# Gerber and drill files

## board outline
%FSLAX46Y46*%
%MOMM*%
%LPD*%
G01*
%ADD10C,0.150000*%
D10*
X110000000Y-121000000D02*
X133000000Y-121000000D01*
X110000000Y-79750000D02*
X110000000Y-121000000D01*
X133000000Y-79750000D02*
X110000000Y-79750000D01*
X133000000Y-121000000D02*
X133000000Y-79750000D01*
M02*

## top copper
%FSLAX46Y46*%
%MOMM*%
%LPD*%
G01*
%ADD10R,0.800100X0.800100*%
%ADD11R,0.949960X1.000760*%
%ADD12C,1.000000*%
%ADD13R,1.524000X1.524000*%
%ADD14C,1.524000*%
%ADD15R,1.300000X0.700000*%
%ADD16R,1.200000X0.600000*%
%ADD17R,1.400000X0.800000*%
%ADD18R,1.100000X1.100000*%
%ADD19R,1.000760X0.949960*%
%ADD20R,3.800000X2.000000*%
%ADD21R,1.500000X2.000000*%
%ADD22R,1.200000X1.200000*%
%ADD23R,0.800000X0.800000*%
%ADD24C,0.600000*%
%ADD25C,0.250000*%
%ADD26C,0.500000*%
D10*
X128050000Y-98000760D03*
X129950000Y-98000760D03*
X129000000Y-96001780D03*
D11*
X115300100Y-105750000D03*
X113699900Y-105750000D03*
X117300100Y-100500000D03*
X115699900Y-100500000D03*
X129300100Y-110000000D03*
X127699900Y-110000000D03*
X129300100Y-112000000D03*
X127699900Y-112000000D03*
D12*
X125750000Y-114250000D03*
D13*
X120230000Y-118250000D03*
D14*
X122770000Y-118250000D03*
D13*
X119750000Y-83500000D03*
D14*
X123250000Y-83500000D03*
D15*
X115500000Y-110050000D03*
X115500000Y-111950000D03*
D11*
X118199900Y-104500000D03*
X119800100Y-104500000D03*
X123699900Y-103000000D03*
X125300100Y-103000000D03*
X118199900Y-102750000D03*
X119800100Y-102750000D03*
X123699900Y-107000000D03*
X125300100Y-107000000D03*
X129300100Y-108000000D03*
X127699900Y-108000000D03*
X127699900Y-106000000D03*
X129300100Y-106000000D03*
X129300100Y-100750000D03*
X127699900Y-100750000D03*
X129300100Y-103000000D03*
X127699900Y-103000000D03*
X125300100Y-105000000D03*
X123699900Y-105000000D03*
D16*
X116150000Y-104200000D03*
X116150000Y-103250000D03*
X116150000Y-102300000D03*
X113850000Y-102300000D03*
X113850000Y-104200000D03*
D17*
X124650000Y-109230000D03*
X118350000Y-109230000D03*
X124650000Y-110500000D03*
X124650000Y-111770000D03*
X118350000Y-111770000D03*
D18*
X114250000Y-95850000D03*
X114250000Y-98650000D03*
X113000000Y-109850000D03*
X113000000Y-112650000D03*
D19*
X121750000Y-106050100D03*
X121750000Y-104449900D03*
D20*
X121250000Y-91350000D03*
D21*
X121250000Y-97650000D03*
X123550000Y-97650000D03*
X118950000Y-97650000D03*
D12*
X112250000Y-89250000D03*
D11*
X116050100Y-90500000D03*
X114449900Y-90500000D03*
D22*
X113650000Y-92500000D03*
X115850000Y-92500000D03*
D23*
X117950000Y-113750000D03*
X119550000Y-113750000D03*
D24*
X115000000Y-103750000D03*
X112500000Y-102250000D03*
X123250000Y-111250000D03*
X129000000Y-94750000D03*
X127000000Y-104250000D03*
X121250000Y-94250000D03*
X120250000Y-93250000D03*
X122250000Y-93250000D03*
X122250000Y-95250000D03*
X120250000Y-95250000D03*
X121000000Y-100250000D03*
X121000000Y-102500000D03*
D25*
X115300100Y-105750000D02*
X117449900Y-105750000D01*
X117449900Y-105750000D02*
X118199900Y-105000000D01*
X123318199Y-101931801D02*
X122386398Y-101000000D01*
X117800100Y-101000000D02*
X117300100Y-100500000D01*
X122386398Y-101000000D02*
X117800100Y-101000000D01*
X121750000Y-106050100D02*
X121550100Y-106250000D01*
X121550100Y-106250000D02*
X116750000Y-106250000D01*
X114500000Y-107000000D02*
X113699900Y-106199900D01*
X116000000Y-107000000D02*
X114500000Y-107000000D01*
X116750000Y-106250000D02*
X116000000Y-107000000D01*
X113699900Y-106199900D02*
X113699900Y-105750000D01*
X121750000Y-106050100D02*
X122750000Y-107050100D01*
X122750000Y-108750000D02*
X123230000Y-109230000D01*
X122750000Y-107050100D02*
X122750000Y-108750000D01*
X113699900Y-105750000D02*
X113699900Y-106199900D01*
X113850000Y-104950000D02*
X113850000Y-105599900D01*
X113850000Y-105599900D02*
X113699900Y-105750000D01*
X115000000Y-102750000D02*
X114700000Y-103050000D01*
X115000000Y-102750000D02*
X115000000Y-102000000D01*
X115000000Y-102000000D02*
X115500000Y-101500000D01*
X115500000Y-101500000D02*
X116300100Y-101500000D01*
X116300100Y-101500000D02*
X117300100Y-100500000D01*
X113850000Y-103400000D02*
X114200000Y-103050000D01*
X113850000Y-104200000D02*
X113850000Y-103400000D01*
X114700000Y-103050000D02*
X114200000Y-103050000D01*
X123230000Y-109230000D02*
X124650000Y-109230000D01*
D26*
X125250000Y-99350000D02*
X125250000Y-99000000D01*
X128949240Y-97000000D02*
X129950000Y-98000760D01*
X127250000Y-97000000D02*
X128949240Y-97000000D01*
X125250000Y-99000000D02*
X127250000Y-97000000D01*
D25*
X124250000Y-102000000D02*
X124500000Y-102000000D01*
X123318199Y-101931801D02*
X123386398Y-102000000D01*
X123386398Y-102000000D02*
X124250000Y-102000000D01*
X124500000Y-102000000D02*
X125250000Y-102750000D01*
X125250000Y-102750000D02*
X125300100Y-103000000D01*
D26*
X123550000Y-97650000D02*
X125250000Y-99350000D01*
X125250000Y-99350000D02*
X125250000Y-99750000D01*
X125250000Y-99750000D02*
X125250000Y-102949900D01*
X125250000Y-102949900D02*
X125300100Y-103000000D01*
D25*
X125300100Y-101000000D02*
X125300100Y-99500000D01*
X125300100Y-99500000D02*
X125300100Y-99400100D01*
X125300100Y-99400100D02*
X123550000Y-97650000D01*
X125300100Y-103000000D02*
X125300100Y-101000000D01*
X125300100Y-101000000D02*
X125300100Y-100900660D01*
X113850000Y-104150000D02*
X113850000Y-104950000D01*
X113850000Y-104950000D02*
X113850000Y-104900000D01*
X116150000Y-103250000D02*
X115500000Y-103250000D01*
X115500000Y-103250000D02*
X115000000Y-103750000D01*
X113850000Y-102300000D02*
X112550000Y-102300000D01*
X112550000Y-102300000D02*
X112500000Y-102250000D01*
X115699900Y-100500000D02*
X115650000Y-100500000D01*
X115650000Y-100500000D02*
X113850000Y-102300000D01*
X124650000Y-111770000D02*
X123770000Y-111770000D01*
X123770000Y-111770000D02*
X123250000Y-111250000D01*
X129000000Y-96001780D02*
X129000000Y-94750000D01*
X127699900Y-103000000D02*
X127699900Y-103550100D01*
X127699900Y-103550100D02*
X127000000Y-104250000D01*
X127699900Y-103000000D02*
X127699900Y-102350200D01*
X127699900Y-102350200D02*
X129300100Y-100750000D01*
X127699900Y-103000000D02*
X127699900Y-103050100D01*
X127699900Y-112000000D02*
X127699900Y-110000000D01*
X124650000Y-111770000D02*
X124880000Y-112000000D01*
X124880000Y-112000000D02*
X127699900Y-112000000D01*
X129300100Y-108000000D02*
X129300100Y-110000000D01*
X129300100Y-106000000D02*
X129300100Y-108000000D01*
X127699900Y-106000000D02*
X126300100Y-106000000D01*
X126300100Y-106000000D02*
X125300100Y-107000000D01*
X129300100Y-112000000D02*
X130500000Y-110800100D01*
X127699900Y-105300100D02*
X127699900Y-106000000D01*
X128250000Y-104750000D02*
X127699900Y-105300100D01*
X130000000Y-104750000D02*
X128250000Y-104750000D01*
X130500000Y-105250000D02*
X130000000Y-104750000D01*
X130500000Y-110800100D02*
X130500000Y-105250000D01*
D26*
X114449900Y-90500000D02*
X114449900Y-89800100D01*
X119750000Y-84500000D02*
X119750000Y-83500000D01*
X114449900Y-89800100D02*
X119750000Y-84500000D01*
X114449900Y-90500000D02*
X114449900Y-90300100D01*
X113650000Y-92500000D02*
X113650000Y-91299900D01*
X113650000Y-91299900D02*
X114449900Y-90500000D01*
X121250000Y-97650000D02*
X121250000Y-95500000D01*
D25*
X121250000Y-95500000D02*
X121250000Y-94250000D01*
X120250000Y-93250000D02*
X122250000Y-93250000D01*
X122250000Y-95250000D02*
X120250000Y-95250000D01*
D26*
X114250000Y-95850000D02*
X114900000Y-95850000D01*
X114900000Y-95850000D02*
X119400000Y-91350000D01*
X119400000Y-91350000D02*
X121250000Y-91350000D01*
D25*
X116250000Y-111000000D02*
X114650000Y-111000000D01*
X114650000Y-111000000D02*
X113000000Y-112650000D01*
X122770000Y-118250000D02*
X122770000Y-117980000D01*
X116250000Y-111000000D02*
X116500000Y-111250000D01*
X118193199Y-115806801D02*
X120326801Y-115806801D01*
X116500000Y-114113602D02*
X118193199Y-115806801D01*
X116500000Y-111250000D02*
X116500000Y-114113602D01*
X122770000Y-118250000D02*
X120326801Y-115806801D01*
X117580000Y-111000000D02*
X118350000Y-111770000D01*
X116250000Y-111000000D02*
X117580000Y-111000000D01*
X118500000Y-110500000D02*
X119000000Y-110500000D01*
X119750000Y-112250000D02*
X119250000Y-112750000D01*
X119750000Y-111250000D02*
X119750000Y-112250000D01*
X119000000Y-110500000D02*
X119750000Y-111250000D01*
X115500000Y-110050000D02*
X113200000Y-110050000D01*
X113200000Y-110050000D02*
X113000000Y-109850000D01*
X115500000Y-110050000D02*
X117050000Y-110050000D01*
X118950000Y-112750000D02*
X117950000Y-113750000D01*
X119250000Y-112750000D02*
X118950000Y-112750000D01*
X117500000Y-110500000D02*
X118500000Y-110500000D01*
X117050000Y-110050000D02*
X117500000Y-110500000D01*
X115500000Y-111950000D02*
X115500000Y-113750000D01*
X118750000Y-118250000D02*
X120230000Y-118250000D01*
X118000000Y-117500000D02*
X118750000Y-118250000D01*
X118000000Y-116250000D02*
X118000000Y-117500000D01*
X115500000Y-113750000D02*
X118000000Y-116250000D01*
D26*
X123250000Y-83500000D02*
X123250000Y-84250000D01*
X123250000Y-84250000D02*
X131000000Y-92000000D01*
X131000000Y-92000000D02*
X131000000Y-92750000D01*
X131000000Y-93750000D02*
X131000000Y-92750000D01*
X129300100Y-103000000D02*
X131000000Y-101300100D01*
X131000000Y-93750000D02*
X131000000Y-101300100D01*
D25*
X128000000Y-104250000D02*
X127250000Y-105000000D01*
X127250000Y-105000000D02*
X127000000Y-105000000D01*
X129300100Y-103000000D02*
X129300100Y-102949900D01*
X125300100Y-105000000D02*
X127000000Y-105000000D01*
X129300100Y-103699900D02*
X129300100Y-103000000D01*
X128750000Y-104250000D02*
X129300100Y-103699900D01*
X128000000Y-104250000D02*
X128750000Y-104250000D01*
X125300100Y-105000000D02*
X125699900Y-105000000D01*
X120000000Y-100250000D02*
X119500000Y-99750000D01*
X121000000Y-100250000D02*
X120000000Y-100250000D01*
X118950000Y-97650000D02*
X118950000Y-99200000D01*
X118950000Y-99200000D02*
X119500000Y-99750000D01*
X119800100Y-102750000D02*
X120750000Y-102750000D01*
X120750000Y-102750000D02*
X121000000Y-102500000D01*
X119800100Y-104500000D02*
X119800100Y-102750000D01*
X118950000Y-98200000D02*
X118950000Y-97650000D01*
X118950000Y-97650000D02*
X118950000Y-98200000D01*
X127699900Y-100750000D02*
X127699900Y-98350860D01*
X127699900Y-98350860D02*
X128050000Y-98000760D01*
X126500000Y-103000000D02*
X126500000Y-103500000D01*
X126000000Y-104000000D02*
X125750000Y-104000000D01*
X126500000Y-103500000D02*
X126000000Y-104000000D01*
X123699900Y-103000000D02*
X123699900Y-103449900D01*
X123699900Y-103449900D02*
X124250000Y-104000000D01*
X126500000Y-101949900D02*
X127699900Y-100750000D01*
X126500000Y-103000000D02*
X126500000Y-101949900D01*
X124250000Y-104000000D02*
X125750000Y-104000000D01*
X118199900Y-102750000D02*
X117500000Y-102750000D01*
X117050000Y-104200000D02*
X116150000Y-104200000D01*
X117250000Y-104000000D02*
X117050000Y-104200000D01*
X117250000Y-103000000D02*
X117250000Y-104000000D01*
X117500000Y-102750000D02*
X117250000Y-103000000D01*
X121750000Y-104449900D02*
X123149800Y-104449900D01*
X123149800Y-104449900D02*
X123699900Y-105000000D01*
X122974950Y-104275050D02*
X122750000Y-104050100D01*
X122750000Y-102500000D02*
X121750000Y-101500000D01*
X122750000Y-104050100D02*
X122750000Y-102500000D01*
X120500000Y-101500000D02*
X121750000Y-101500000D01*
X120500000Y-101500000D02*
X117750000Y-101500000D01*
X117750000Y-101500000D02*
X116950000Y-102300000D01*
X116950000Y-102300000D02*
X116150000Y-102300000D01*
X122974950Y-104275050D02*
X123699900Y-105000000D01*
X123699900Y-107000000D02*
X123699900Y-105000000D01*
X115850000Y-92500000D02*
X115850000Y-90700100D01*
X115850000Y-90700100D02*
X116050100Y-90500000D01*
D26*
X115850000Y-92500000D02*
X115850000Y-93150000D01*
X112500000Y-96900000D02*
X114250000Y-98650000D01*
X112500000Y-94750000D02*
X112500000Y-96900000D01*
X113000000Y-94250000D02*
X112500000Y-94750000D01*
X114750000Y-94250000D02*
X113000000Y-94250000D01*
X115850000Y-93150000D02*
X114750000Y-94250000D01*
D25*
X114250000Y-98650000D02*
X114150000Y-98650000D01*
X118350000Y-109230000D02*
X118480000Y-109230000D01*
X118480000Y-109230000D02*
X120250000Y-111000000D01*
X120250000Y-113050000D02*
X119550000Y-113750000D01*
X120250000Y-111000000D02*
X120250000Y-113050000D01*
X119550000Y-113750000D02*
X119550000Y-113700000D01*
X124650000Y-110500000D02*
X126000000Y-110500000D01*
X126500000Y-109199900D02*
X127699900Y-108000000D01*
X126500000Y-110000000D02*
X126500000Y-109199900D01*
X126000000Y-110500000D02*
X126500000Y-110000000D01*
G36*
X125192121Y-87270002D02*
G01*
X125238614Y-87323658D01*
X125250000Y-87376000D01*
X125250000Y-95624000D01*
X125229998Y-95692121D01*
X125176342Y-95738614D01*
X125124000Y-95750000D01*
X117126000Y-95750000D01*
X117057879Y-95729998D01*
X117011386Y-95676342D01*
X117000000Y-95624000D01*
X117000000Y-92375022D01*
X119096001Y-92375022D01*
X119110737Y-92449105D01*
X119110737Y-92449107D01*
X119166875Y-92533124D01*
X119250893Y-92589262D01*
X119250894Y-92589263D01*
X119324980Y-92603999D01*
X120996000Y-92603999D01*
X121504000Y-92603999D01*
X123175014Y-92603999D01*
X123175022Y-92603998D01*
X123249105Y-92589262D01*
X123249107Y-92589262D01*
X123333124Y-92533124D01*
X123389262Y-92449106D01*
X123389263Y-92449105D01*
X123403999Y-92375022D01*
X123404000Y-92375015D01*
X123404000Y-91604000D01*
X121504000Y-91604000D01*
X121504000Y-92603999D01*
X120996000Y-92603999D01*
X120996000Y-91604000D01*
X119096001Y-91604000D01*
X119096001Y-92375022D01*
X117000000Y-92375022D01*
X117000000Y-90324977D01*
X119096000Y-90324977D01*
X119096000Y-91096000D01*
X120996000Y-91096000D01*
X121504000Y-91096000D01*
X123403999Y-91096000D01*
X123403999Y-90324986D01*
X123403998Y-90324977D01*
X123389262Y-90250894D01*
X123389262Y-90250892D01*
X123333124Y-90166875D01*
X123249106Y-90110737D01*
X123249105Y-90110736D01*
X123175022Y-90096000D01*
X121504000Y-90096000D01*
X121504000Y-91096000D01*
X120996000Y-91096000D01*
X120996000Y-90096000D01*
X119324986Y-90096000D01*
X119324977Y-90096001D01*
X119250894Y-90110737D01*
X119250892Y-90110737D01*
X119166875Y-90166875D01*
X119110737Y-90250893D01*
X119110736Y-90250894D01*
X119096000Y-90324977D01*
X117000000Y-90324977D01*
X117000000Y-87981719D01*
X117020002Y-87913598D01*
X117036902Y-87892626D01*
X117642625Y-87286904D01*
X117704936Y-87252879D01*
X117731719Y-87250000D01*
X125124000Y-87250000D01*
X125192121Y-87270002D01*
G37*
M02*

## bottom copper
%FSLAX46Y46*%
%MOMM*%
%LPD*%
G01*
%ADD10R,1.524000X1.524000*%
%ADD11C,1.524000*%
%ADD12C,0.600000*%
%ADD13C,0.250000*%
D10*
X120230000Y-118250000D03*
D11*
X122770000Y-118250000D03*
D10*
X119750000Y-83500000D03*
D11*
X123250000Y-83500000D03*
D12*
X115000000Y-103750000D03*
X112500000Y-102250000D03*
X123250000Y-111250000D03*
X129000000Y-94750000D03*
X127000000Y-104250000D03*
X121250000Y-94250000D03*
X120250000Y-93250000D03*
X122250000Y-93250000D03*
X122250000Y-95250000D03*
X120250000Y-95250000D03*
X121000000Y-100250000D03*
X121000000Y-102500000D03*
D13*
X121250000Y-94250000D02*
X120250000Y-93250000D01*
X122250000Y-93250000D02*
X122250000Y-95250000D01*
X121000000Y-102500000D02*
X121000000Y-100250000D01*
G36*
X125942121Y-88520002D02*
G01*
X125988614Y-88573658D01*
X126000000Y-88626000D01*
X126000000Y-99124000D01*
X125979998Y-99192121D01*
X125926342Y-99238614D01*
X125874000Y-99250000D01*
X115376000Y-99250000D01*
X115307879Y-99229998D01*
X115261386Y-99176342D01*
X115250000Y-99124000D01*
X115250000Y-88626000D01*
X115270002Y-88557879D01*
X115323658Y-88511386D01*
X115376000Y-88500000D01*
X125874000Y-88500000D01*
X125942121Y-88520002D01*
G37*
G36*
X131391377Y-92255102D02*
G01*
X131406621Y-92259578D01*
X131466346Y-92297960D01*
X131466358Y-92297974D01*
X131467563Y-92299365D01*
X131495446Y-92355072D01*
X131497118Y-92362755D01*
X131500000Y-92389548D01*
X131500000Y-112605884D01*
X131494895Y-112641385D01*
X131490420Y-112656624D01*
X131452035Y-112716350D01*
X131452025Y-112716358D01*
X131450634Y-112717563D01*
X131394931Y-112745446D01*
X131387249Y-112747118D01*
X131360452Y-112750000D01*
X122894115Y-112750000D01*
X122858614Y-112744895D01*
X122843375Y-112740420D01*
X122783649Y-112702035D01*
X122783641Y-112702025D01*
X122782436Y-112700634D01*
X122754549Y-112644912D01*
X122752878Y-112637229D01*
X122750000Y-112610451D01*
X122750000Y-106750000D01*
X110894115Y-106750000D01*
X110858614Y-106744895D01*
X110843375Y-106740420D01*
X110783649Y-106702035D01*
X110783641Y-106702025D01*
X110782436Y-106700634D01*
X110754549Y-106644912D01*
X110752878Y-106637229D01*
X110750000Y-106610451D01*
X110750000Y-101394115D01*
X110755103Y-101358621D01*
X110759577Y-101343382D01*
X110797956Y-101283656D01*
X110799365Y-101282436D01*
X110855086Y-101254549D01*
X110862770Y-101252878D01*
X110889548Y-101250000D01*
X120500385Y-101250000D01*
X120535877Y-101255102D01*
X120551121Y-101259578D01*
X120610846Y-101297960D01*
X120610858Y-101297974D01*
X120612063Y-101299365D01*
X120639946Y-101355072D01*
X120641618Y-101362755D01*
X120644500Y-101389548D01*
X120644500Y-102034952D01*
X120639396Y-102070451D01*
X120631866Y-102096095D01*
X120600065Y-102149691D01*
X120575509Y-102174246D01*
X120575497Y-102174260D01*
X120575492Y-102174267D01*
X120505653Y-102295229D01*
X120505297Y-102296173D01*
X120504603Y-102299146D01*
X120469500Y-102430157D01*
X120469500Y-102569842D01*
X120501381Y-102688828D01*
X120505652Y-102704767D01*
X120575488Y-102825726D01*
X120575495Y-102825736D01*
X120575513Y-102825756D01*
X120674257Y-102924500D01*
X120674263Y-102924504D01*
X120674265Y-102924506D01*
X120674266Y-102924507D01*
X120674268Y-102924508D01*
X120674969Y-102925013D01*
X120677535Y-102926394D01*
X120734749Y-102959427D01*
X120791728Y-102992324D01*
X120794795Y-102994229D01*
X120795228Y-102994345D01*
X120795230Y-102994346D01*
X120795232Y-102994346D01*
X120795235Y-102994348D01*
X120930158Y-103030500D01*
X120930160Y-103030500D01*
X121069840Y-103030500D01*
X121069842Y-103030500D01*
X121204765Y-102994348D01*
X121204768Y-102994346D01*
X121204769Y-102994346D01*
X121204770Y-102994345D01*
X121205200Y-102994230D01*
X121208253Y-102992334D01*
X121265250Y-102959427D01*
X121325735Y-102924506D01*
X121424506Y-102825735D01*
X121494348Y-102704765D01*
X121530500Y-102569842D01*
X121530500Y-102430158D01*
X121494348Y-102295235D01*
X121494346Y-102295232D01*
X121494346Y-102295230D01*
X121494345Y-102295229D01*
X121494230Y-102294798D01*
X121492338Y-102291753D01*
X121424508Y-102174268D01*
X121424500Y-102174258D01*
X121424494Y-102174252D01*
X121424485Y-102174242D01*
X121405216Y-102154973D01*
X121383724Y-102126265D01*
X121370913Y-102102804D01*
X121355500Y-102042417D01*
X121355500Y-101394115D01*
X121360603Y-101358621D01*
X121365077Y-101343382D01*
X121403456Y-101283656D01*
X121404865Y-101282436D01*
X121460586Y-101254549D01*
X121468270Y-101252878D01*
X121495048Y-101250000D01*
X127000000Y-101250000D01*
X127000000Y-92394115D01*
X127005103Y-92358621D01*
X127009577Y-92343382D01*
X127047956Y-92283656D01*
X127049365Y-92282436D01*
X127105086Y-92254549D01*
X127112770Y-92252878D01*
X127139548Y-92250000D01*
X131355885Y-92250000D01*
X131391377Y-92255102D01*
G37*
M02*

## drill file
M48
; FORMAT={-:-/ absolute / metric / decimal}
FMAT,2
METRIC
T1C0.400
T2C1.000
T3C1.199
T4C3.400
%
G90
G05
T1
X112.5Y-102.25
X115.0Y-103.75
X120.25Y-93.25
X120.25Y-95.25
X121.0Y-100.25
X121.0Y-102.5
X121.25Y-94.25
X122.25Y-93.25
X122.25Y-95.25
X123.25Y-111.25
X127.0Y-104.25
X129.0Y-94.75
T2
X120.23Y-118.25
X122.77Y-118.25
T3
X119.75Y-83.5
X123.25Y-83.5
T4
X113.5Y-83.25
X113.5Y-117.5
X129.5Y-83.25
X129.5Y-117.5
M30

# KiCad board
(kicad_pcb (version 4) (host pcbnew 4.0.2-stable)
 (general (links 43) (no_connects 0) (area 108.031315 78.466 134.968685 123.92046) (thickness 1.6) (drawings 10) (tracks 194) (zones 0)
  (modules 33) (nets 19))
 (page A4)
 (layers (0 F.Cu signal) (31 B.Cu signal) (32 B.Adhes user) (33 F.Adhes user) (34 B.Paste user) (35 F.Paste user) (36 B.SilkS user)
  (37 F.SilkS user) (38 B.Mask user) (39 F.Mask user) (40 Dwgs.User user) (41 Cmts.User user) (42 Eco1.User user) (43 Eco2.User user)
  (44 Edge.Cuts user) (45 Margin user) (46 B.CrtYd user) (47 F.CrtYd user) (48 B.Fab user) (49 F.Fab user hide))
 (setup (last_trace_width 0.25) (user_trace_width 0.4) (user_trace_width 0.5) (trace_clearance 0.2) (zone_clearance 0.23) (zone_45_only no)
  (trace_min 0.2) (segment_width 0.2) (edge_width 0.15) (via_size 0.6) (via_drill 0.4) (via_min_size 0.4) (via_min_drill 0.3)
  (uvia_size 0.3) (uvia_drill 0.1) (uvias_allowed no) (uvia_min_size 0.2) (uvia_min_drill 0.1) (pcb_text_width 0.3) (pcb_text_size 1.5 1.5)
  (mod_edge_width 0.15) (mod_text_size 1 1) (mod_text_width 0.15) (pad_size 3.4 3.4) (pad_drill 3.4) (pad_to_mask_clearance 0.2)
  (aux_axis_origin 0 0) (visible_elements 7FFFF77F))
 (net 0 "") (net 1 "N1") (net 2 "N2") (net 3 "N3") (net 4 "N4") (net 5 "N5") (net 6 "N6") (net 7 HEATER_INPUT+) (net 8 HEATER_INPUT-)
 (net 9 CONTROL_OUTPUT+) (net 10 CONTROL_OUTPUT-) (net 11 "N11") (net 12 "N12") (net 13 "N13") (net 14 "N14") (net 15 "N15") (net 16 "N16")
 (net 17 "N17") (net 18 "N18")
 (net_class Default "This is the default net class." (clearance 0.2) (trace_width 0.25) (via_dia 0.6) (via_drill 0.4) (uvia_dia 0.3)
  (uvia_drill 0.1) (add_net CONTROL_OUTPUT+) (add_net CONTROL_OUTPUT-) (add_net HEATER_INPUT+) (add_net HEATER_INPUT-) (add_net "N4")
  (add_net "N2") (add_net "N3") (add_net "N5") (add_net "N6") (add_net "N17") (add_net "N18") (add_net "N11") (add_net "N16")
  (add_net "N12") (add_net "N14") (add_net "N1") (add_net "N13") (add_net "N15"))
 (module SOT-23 (layer F.Cu) (at 129 97)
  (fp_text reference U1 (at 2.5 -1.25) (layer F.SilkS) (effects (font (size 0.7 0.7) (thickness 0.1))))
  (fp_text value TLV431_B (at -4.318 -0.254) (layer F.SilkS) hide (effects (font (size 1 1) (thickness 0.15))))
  (pad 1 smd rect (at -0.95 1.00076) (size 0.8001 0.8001) (layers F.Cu F.Paste F.Mask) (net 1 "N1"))
  (pad 2 smd rect (at 0.95 1.00076) (size 0.8001 0.8001) (layers F.Cu F.Paste F.Mask) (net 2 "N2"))
  (pad 3 smd rect (at 0 -0.99822) (size 0.8001 0.8001) (layers F.Cu F.Paste F.Mask) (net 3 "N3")))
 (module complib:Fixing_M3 (layer F.Cu) (at 129.5 117.5)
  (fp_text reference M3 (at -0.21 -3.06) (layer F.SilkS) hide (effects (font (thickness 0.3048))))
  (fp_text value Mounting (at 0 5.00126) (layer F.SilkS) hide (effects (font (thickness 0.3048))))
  (pad "" np_thru_hole circle (at 0 0) (size 3.4 3.4) (drill 3.4) (layers *.Cu *.Mask F.SilkS)))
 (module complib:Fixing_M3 (layer F.Cu) (at 113.5 83.25)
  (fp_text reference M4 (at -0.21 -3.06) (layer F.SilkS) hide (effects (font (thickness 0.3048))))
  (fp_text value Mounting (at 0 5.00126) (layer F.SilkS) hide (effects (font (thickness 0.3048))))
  (pad "" np_thru_hole circle (at 0 0) (size 3.4 3.4) (drill 3.4) (layers *.Cu *.Mask F.SilkS)))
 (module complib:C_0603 (layer F.Cu) (at 114.5 105.75)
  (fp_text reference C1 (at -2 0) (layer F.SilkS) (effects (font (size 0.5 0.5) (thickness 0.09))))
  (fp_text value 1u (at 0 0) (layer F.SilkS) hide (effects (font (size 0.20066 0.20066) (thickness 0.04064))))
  (pad 1 smd rect (at 0.8001 0) (size 0.94996 1.00076) (layers F.Cu F.Paste F.Mask) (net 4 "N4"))
  (pad 2 smd rect (at -0.8001 0) (size 0.94996 1.00076) (layers F.Cu F.Paste F.Mask) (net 2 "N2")))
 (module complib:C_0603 (layer F.Cu) (at 116.5 100.5)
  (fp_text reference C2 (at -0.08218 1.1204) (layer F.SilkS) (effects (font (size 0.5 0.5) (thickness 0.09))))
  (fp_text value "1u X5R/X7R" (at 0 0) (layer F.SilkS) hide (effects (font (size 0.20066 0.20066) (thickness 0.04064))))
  (pad 1 smd rect (at 0.8001 0) (size 0.94996 1.00076) (layers F.Cu F.Paste F.Mask) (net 2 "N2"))
  (pad 2 smd rect (at -0.8001 0) (size 0.94996 1.00076) (layers F.Cu F.Paste F.Mask) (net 3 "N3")))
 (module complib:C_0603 (layer F.Cu) (at 128.5 110)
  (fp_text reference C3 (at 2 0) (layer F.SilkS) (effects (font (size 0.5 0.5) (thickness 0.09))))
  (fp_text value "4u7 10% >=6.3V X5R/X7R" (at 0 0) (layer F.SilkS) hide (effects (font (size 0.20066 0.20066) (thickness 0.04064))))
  (pad 1 smd rect (at 0.8001 0) (size 0.94996 1.00076) (layers F.Cu F.Paste F.Mask) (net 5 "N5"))
  (pad 2 smd rect (at -0.8001 0) (size 0.94996 1.00076) (layers F.Cu F.Paste F.Mask) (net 3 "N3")))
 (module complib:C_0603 (layer F.Cu) (at 128.5 112)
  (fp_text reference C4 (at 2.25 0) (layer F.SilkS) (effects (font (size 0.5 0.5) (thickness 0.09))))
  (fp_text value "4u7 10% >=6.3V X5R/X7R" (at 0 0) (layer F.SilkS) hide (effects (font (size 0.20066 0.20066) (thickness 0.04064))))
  (pad 1 smd rect (at 0.8001 0) (size 0.94996 1.00076) (layers F.Cu F.Paste F.Mask) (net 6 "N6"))
  (pad 2 smd rect (at -0.8001 0) (size 0.94996 1.00076) (layers F.Cu F.Paste F.Mask) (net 3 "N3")))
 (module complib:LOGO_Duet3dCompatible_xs (layer B.Cu) (at 117.25 101.75 270)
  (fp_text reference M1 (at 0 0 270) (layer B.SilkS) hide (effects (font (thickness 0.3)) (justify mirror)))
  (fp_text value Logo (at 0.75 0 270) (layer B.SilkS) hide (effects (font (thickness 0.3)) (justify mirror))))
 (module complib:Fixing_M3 (layer F.Cu) (at 129.5 83.25)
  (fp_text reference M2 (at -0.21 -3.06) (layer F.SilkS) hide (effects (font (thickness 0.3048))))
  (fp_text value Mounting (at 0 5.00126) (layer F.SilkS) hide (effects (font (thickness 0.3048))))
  (pad "" np_thru_hole circle (at 0 0) (size 3.4 3.4) (drill 3.4) (layers *.Cu *.Mask F.SilkS)))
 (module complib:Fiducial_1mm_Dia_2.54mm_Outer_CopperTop (layer F.Cu) (at 125.75 114.25)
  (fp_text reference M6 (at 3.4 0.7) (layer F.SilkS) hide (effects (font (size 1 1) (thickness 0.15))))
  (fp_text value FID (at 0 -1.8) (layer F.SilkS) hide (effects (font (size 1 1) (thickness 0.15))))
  (pad ~ smd circle (at 0 0) (size 1 1) (layers F.Cu F.Mask) (solder_mask_margin 0.77) (clearance 0.77)))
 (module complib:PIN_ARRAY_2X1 (layer F.Cu) (at 121.5 118.25)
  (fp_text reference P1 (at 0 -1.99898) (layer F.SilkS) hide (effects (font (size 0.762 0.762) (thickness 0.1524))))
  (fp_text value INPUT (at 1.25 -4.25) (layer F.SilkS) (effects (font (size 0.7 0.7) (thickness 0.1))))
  (pad 1 thru_hole rect (at -1.27 0) (size 1.524 1.524) (drill 1) (layers *.Cu *.Mask F.SilkS) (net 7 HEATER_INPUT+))
  (pad 2 thru_hole circle (at 1.27 0) (size 1.524 1.524) (drill 1) (layers *.Cu *.Mask F.SilkS) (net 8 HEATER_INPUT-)))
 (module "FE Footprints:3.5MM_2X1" (layer F.Cu) (at 121.5 83.5)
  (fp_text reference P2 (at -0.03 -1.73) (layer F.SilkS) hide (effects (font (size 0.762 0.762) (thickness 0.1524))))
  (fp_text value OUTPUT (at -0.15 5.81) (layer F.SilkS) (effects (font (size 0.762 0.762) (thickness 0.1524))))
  (pad 1 thru_hole rect (at -1.75 0) (size 1.524 1.524) (drill 1.19888) (layers *.Cu *.Mask F.SilkS) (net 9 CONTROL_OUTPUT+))
  (pad 2 thru_hole circle (at 1.75 0) (size 1.524 1.524) (drill 1.19888) (layers *.Cu *.Mask F.SilkS) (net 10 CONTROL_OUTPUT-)))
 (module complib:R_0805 (layer F.Cu) (at 115.5 111 270)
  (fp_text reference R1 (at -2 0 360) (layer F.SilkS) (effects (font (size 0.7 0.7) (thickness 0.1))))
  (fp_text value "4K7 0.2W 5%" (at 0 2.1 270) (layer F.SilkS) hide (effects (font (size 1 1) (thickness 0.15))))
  (pad 1 smd rect (at -0.95 0 270) (size 0.7 1.3) (layers F.Cu F.Paste F.Mask) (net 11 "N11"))
  (pad 2 smd rect (at 0.95 0 270) (size 0.7 1.3) (layers F.Cu F.Paste F.Mask) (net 7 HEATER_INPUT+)))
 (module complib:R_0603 (layer F.Cu) (at 119 104.5)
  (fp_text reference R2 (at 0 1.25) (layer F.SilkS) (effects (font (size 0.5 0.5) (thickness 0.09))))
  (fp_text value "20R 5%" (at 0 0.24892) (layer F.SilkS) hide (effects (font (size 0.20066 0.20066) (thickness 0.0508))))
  (pad 1 smd rect (at -0.8001 0) (size 0.94996 1.00076) (layers F.Cu F.Paste F.Mask) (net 4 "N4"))
  (pad 2 smd rect (at 0.8001 0) (size 0.94996 1.00076) (layers F.Cu F.Paste F.Mask) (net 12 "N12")))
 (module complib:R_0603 (layer F.Cu) (at 124.5 103)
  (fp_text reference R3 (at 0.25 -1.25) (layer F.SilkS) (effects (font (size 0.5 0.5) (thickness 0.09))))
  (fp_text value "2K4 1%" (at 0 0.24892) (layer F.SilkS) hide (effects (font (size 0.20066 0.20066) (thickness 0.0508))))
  (pad 1 smd rect (at -0.8001 0) (size 0.94996 1.00076) (layers F.Cu F.Paste F.Mask) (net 1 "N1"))
  (pad 2 smd rect (at 0.8001 0) (size 0.94996 1.00076) (layers F.Cu F.Paste F.Mask) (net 2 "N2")))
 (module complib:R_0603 (layer F.Cu) (at 119 102.75)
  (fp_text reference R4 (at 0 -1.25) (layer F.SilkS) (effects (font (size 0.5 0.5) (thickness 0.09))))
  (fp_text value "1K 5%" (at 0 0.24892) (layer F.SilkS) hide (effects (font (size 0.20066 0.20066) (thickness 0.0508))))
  (pad 1 smd rect (at -0.8001 0) (size 0.94996 1.00076) (layers F.Cu F.Paste F.Mask) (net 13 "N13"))
  (pad 2 smd rect (at 0.8001 0) (size 0.94996 1.00076) (layers F.Cu F.Paste F.Mask) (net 12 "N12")))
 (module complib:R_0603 (layer F.Cu) (at 124.5 107)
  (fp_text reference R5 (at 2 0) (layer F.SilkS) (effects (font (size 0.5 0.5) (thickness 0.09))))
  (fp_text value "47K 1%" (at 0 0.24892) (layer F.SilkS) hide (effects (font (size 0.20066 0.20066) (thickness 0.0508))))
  (pad 1 smd rect (at -0.8001 0) (size 0.94996 1.00076) (layers F.Cu F.Paste F.Mask) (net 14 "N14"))
  (pad 2 smd rect (at 0.8001 0) (size 0.94996 1.00076) (layers F.Cu F.Paste F.Mask) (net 6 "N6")))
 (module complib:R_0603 (layer F.Cu) (at 128.5 108 180)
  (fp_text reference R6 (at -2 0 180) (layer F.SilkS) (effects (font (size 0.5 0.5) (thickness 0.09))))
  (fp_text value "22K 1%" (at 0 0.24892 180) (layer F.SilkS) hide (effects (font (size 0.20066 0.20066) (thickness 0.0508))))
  (pad 1 smd rect (at -0.8001 0 180) (size 0.94996 1.00076) (layers F.Cu F.Paste F.Mask) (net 5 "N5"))
  (pad 2 smd rect (at 0.8001 0 180) (size 0.94996 1.00076) (layers F.Cu F.Paste F.Mask) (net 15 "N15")))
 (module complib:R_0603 (layer F.Cu) (at 128.5 106)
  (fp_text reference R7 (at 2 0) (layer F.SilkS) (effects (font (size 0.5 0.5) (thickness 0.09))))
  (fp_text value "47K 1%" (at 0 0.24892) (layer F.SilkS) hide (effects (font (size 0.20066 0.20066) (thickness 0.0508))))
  (pad 1 smd rect (at -0.8001 0) (size 0.94996 1.00076) (layers F.Cu F.Paste F.Mask) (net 6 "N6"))
  (pad 2 smd rect (at 0.8001 0) (size 0.94996 1.00076) (layers F.Cu F.Paste F.Mask) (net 5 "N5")))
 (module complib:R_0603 (layer F.Cu) (at 128.5 100.75 180)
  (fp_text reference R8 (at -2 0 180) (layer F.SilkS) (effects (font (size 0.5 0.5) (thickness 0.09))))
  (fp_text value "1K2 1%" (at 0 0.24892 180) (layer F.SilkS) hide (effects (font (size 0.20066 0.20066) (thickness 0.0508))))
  (pad 1 smd rect (at -0.8001 0 180) (size 0.94996 1.00076) (layers F.Cu F.Paste F.Mask) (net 3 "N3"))
  (pad 2 smd rect (at 0.8001 0 180) (size 0.94996 1.00076) (layers F.Cu F.Paste F.Mask) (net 1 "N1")))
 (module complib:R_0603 (layer F.Cu) (at 128.5 103 180)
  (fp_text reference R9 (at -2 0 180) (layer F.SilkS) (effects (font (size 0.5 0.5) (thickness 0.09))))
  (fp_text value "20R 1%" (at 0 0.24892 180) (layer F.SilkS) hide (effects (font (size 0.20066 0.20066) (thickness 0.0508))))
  (pad 1 smd rect (at -0.8001 0 180) (size 0.94996 1.00076) (layers F.Cu F.Paste F.Mask) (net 10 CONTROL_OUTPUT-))
  (pad 2 smd rect (at 0.8001 0 180) (size 0.94996 1.00076) (layers F.Cu F.Paste F.Mask) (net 3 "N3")))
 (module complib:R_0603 (layer F.Cu) (at 124.5 105 180)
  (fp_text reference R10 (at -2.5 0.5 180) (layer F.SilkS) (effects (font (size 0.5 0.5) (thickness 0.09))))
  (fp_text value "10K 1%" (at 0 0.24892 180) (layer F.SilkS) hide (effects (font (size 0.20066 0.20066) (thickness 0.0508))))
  (pad 1 smd rect (at -0.8001 0 180) (size 0.94996 1.00076) (layers F.Cu F.Paste F.Mask) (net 10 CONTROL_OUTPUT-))
  (pad 2 smd rect (at 0.8001 0 180) (size 0.94996 1.00076) (layers F.Cu F.Paste F.Mask) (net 14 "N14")))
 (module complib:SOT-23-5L (layer F.Cu) (at 115 103.25 180)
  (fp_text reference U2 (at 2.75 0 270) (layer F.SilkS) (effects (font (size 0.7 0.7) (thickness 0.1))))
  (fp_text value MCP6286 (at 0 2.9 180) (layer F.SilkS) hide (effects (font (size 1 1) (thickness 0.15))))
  (pad 1 smd rect (at -1.15 -0.95 180) (size 1.2 0.6) (layers F.Cu F.Paste F.Mask) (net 13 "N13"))
  (pad 2 smd rect (at -1.15 0 180) (size 1.2 0.6) (layers F.Cu F.Paste F.Mask) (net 3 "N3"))
  (pad 3 smd rect (at -1.15 0.95 180) (size 1.2 0.6) (layers F.Cu F.Paste F.Mask) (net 14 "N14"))
  (pad 4 smd rect (at 1.15 0.95 180) (size 1.2 0.6) (layers F.Cu F.Paste F.Mask) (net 3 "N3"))
  (pad 5 smd rect (at 1.15 -0.95 180) (size 1.2 0.6) (layers F.Cu F.Paste F.Mask) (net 2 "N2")))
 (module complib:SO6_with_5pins (layer F.Cu) (at 121.5 110.5 270)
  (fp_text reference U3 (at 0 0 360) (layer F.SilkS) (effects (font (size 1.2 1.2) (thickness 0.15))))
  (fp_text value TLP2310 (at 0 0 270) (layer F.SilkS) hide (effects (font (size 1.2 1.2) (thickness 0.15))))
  (pad 6 smd rect (at -1.27 -3.15 270) (size 0.8 1.4) (layers F.Cu F.Paste F.Mask) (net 2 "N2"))
  (pad 1 smd rect (at -1.27 3.15 270) (size 0.8 1.4) (layers F.Cu F.Paste F.Mask) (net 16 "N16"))
  (pad 5 smd rect (at 0 -3.15 270) (size 0.8 1.4) (layers F.Cu F.Paste F.Mask) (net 15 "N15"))
  (pad 4 smd rect (at 1.27 -3.15 270) (size 0.8 1.4) (layers F.Cu F.Paste F.Mask) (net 3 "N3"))
  (pad 3 smd rect (at 1.27 3.15 270) (size 0.8 1.4) (layers F.Cu F.Paste F.Mask) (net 8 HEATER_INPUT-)))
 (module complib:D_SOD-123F (layer F.Cu) (at 114.25 97.25 270)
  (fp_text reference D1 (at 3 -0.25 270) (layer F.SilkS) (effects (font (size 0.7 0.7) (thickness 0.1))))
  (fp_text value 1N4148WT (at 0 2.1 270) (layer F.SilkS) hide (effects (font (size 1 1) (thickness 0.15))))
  (pad 1 smd rect (at -1.4 0 270) (size 1.1 1.1) (layers F.Cu F.Paste F.Mask) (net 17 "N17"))
  (pad 2 smd rect (at 1.4 0 270) (size 1.1 1.1) (layers F.Cu F.Paste F.Mask) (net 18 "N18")))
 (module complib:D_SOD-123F (layer F.Cu) (at 113 111.25 270)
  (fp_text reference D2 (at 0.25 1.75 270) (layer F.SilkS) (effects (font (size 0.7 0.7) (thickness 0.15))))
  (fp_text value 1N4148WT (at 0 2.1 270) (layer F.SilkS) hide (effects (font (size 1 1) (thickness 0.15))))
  (pad 1 smd rect (at -1.4 0 270) (size 1.1 1.1) (layers F.Cu F.Paste F.Mask) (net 11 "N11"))
  (pad 2 smd rect (at 1.4 0 270) (size 1.1 1.1) (layers F.Cu F.Paste F.Mask) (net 8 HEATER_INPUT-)))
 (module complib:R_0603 (layer F.Cu) (at 121.75 105.25 90)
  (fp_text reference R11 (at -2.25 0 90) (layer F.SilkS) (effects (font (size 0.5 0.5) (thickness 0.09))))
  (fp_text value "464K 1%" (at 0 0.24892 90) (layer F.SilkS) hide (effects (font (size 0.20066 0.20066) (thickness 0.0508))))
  (pad 1 smd rect (at -0.8001 0 90) (size 0.94996 1.00076) (layers F.Cu F.Paste F.Mask) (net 2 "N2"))
  (pad 2 smd rect (at 0.8001 0 90) (size 0.94996 1.00076) (layers F.Cu F.Paste F.Mask) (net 14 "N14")))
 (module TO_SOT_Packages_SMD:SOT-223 (layer F.Cu) (at 121.25 94.5 90)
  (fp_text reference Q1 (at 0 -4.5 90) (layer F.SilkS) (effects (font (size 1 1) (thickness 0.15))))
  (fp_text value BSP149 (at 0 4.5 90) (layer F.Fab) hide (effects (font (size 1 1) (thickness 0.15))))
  (pad 4 smd rect (at 3.15 0 90) (size 2 3.8) (layers F.Cu F.Paste F.Mask) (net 17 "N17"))
  (pad 2 smd rect (at -3.15 0 90) (size 2 1.5) (layers F.Cu F.Paste F.Mask) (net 17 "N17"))
  (pad 3 smd rect (at -3.15 2.3 90) (size 2 1.5) (layers F.Cu F.Paste F.Mask) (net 2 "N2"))
  (pad 1 smd rect (at -3.15 -2.3 90) (size 2 1.5) (layers F.Cu F.Paste F.Mask) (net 12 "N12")))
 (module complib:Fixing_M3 (layer F.Cu) (at 113.5 117.5)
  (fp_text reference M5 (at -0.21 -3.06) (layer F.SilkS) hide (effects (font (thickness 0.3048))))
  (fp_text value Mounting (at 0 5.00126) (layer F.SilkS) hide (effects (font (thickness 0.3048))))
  (pad "" np_thru_hole circle (at 0 0) (size 3.4 3.4) (drill 3.4) (layers *.Cu *.Mask F.SilkS)))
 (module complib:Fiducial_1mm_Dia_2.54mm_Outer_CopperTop (layer F.Cu) (at 112.25 89.25)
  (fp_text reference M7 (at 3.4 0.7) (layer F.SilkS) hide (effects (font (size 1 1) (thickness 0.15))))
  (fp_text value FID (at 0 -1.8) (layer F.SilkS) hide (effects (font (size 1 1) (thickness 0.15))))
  (pad ~ smd circle (at 0 0) (size 1 1) (layers F.Cu F.Mask) (solder_mask_margin 0.77) (clearance 0.77)))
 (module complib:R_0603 (layer F.Cu) (at 115.25 90.5 180)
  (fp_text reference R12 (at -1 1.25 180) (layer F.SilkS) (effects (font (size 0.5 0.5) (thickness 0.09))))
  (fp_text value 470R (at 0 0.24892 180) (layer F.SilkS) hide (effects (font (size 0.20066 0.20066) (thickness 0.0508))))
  (pad 1 smd rect (at -0.8001 0 180) (size 0.94996 1.00076) (layers F.Cu F.Paste F.Mask) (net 18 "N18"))
  (pad 2 smd rect (at 0.8001 0 180) (size 0.94996 1.00076) (layers F.Cu F.Paste F.Mask) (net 9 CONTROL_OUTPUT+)))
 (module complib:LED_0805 (layer F.Cu) (at 114.75 92.5 180)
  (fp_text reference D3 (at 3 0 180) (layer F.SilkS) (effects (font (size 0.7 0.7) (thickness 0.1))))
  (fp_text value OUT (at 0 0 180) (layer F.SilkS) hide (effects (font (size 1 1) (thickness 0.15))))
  (pad 2 smd rect (at 1.1 0) (size 1.2 1.2) (layers F.Cu F.Paste F.Mask) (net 9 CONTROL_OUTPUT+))
  (pad 1 smd rect (at -1.1 0) (size 1.2 1.2) (layers F.Cu F.Paste F.Mask) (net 18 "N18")))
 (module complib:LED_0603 (layer F.Cu) (at 118.75 113.75 180)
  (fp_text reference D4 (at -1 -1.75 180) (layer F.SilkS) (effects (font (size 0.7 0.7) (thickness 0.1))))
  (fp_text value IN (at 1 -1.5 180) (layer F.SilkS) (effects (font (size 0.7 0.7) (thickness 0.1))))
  (pad 2 smd rect (at 0.8 0) (size 0.8 0.8) (layers F.Cu F.Paste F.Mask) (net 11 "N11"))
  (pad 1 smd rect (at -0.8 0) (size 0.8 0.8) (layers F.Cu F.Paste F.Mask) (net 16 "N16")))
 (gr_line (start 110 121) (end 133 121) (angle 90) (layer Edge.Cuts) (width 0.15))
 (gr_line (start 110 79.75) (end 110 121) (angle 90) (layer Edge.Cuts) (width 0.15))
 (gr_line (start 133 79.75) (end 110 79.75) (angle 90) (layer Edge.Cuts) (width 0.15))
 (gr_line (start 133 121) (end 133 79.75) (angle 90) (layer Edge.Cuts) (width 0.15))
 (segment (start 115.3001 105.75) (end 117.4499 105.75) (width 0.25) (layer F.Cu) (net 4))
 (segment (start 117.4499 105.75) (end 118.1999 105) (width 0.25) (layer F.Cu) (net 4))
 (segment (start 123.318199 101.931801) (end 122.386398 101) (width 0.25) (layer F.Cu) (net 2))
 (segment (start 117.8001 101) (end 117.3001 100.5) (width 0.25) (layer F.Cu) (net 2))
 (segment (start 122.386398 101) (end 117.8001 101) (width 0.25) (layer F.Cu) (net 2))
 (segment (start 121.75 106.0501) (end 121.5501 106.25) (width 0.25) (layer F.Cu) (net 2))
 (segment (start 121.5501 106.25) (end 116.75 106.25) (width 0.25) (layer F.Cu) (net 2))
 (segment (start 114.5 107) (end 113.6999 106.1999) (width 0.25) (layer F.Cu) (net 2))
 (segment (start 116 107) (end 114.5 107) (width 0.25) (layer F.Cu) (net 2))
 (segment (start 116.75 106.25) (end 116 107) (width 0.25) (layer F.Cu) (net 2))
 (segment (start 113.6999 106.1999) (end 113.6999 105.75) (width 0.25) (layer F.Cu) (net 2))
 (segment (start 121.75 106.0501) (end 122.75 107.0501) (width 0.25) (layer F.Cu) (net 2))
 (segment (start 122.75 108.75) (end 123.23 109.23) (width 0.25) (layer F.Cu) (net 2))
 (segment (start 122.75 107.0501) (end 122.75 108.75) (width 0.25) (layer F.Cu) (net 2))
 (segment (start 113.6999 105.75) (end 113.6999 106.1999) (width 0.25) (layer F.Cu) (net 2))
 (segment (start 113.85 104.95) (end 113.85 105.5999) (width 0.25) (layer F.Cu) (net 2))
 (segment (start 113.85 105.5999) (end 113.6999 105.75) (width 0.25) (layer F.Cu) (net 2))
 (segment (start 115 102.75) (end 114.7 103.05) (width 0.25) (layer F.Cu) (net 2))
 (segment (start 115 102.75) (end 115 102) (width 0.25) (layer F.Cu) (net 2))
 (segment (start 115 102) (end 115.5 101.5) (width 0.25) (layer F.Cu) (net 2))
 (segment (start 115.5 101.5) (end 116.3001 101.5) (width 0.25) (layer F.Cu) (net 2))
 (segment (start 116.3001 101.5) (end 117.3001 100.5) (width 0.25) (layer F.Cu) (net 2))
 (segment (start 113.85 103.4) (end 114.2 103.05) (width 0.25) (layer F.Cu) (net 2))
 (segment (start 113.85 104.2) (end 113.85 103.4) (width 0.25) (layer F.Cu) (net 2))
 (segment (start 114.7 103.05) (end 114.2 103.05) (width 0.25) (layer F.Cu) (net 2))
 (segment (start 123.23 109.23) (end 124.65 109.23) (width 0.25) (layer F.Cu) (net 2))
 (segment (start 125.25 99.35) (end 125.25 99) (width 0.5) (layer F.Cu) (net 2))
 (segment (start 128.94924 97) (end 129.95 98.00076) (width 0.5) (layer F.Cu) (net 2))
 (segment (start 127.25 97) (end 128.94924 97) (width 0.5) (layer F.Cu) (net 2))
 (segment (start 125.25 99) (end 127.25 97) (width 0.5) (layer F.Cu) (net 2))
 (segment (start 124.25 102) (end 124.5 102) (width 0.25) (layer F.Cu) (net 2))
 (segment (start 123.318199 101.931801) (end 123.386398 102) (width 0.25) (layer F.Cu) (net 2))
 (segment (start 123.386398 102) (end 124.25 102) (width 0.25) (layer F.Cu) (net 2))
 (segment (start 124.5 102) (end 125.25 102.75) (width 0.25) (layer F.Cu) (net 2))
 (segment (start 125.25 102.75) (end 125.3001 103) (width 0.25) (layer F.Cu) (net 2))
 (segment (start 123.55 97.65) (end 125.25 99.35) (width 0.5) (layer F.Cu) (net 2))
 (segment (start 125.25 99.35) (end 125.25 99.75) (width 0.5) (layer F.Cu) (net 2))
 (segment (start 125.25 99.75) (end 125.25 102.9499) (width 0.5) (layer F.Cu) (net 2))
 (segment (start 125.25 102.9499) (end 125.3001 103) (width 0.5) (layer F.Cu) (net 2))
 (segment (start 125.3001 101) (end 125.3001 99.5) (width 0.25) (layer F.Cu) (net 2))
 (segment (start 125.3001 99.5) (end 125.3001 99.4001) (width 0.25) (layer F.Cu) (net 2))
 (segment (start 125.3001 99.4001) (end 123.55 97.65) (width 0.25) (layer F.Cu) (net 2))
 (segment (start 125.3001 103) (end 125.3001 101) (width 0.25) (layer F.Cu) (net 2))
 (segment (start 125.3001 101) (end 125.3001 100.90066) (width 0.25) (layer F.Cu) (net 2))
 (segment (start 113.85 104.15) (end 113.85 104.95) (width 0.25) (layer F.Cu) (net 2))
 (segment (start 113.85 104.95) (end 113.85 104.9) (width 0.25) (layer F.Cu) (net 2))
 (segment (start 116.15 103.25) (end 115.5 103.25) (width 0.25) (layer F.Cu) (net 3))
 (via (at 115 103.75) (size 0.6) (drill 0.4) (layers F.Cu B.Cu) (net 3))
 (segment (start 115.5 103.25) (end 115 103.75) (width 0.25) (layer F.Cu) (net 3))
 (segment (start 113.85 102.3) (end 112.55 102.3) (width 0.25) (layer F.Cu) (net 3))
 (via (at 112.5 102.25) (size 0.6) (drill 0.4) (layers F.Cu B.Cu) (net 3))
 (segment (start 112.55 102.3) (end 112.5 102.25) (width 0.25) (layer F.Cu) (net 3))
 (segment (start 115.6999 100.5) (end 115.65 100.5) (width 0.25) (layer F.Cu) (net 3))
 (segment (start 115.65 100.5) (end 113.85 102.3) (width 0.25) (layer F.Cu) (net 3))
 (segment (start 124.65 111.77) (end 123.77 111.77) (width 0.25) (layer F.Cu) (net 3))
 (via (at 123.25 111.25) (size 0.6) (drill 0.4) (layers F.Cu B.Cu) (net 3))
 (segment (start 123.77 111.77) (end 123.25 111.25) (width 0.25) (layer F.Cu) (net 3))
 (segment (start 129 96.00178) (end 129 94.75) (width 0.25) (layer F.Cu) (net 3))
 (via (at 129 94.75) (size 0.6) (drill 0.4) (layers F.Cu B.Cu) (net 3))
 (segment (start 127.6999 103) (end 127.6999 103.5501) (width 0.25) (layer F.Cu) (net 3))
 (segment (start 127.6999 103.5501) (end 127 104.25) (width 0.25) (layer F.Cu) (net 3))
 (via (at 127 104.25) (size 0.6) (drill 0.4) (layers F.Cu B.Cu) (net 3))
 (segment (start 127.6999 103) (end 127.6999 102.3502) (width 0.25) (layer F.Cu) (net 3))
 (segment (start 127.6999 102.3502) (end 129.3001 100.75) (width 0.25) (layer F.Cu) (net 3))
 (segment (start 127.6999 103) (end 127.6999 103.0501) (width 0.25) (layer F.Cu) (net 3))
 (segment (start 127.6999 112) (end 127.6999 110) (width 0.25) (layer F.Cu) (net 3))
 (segment (start 124.65 111.77) (end 124.88 112) (width 0.25) (layer F.Cu) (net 3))
 (segment (start 124.88 112) (end 127.6999 112) (width 0.25) (layer F.Cu) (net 3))
 (segment (start 129.3001 108) (end 129.3001 110) (width 0.25) (layer F.Cu) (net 5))
 (segment (start 129.3001 106) (end 129.3001 108) (width 0.25) (layer F.Cu) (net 5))
 (segment (start 127.6999 106) (end 126.3001 106) (width 0.25) (layer F.Cu) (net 6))
 (segment (start 126.3001 106) (end 125.3001 107) (width 0.25) (layer F.Cu) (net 6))
 (segment (start 129.3001 112) (end 130.5 110.8001) (width 0.25) (layer F.Cu) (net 6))
 (segment (start 127.6999 105.3001) (end 127.6999 106) (width 0.25) (layer F.Cu) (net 6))
 (segment (start 128.25 104.75) (end 127.6999 105.3001) (width 0.25) (layer F.Cu) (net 6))
 (segment (start 130 104.75) (end 128.25 104.75) (width 0.25) (layer F.Cu) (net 6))
 (segment (start 130.5 105.25) (end 130 104.75) (width 0.25) (layer F.Cu) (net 6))
 (segment (start 130.5 110.8001) (end 130.5 105.25) (width 0.25) (layer F.Cu) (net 6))
 (segment (start 114.4499 90.5) (end 114.4499 89.8001) (width 0.5) (layer F.Cu) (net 9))
 (segment (start 119.75 84.5) (end 119.75 83.5) (width 0.5) (layer F.Cu) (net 9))
 (segment (start 114.4499 89.8001) (end 119.75 84.5) (width 0.5) (layer F.Cu) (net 9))
 (segment (start 114.4499 90.5) (end 114.4499 90.3001) (width 0.5) (layer F.Cu) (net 9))
 (segment (start 113.65 92.5) (end 113.65 91.2999) (width 0.5) (layer F.Cu) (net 9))
 (segment (start 113.65 91.2999) (end 114.4499 90.5) (width 0.5) (layer F.Cu) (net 9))
 (segment (start 121.25 97.65) (end 121.25 95.5) (width 0.5) (layer F.Cu) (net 17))
 (segment (start 121.25 95.5) (end 121.25 94.25) (width 0.25) (layer F.Cu) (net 17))
 (via (at 121.25 94.25) (size 0.6) (drill 0.4) (layers F.Cu B.Cu) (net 17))
 (segment (start 121.25 94.25) (end 120.25 93.25) (width 0.25) (layer B.Cu) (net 17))
 (via (at 120.25 93.25) (size 0.6) (drill 0.4) (layers F.Cu B.Cu) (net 17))
 (segment (start 120.25 93.25) (end 122.25 93.25) (width 0.25) (layer F.Cu) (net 17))
 (via (at 122.25 93.25) (size 0.6) (drill 0.4) (layers F.Cu B.Cu) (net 17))
 (segment (start 122.25 93.25) (end 122.25 95.25) (width 0.25) (layer B.Cu) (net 17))
 (via (at 122.25 95.25) (size 0.6) (drill 0.4) (layers F.Cu B.Cu) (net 17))
 (segment (start 122.25 95.25) (end 120.25 95.25) (width 0.25) (layer F.Cu) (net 17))
 (via (at 120.25 95.25) (size 0.6) (drill 0.4) (layers F.Cu B.Cu) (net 17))
 (segment (start 114.25 95.85) (end 114.9 95.85) (width 0.5) (layer F.Cu) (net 17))
 (segment (start 114.9 95.85) (end 119.4 91.35) (width 0.5) (layer F.Cu) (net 17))
 (segment (start 119.4 91.35) (end 121.25 91.35) (width 0.5) (layer F.Cu) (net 17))
 (segment (start 116.25 111) (end 114.65 111) (width 0.25) (layer F.Cu) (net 8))
 (segment (start 114.65 111) (end 113 112.65) (width 0.25) (layer F.Cu) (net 8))
 (segment (start 122.77 118.25) (end 122.77 117.98) (width 0.25) (layer F.Cu) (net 8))
 (segment (start 116.25 111) (end 116.5 111.25) (width 0.25) (layer F.Cu) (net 8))
 (segment (start 118.193199 115.806801) (end 120.326801 115.806801) (width 0.25) (layer F.Cu) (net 8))
 (segment (start 116.5 114.113602) (end 118.193199 115.806801) (width 0.25) (layer F.Cu) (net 8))
 (segment (start 116.5 111.25) (end 116.5 114.113602) (width 0.25) (layer F.Cu) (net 8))
 (segment (start 122.77 118.25) (end 120.326801 115.806801) (width 0.25) (layer F.Cu) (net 8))
 (segment (start 117.58 111) (end 118.35 111.77) (width 0.25) (layer F.Cu) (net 8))
 (segment (start 116.25 111) (end 117.58 111) (width 0.25) (layer F.Cu) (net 8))
 (segment (start 118.5 110.5) (end 119 110.5) (width 0.25) (layer F.Cu) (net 11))
 (segment (start 119.75 112.25) (end 119.25 112.75) (width 0.25) (layer F.Cu) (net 11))
 (segment (start 119.75 111.25) (end 119.75 112.25) (width 0.25) (layer F.Cu) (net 11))
 (segment (start 119 110.5) (end 119.75 111.25) (width 0.25) (layer F.Cu) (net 11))
 (segment (start 115.5 110.05) (end 113.2 110.05) (width 0.25) (layer F.Cu) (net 11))
 (segment (start 113.2 110.05) (end 113 109.85) (width 0.25) (layer F.Cu) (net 11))
 (segment (start 115.5 110.05) (end 117.05 110.05) (width 0.25) (layer F.Cu) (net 11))
 (segment (start 118.95 112.75) (end 117.95 113.75) (width 0.25) (layer F.Cu) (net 11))
 (segment (start 119.25 112.75) (end 118.95 112.75) (width 0.25) (layer F.Cu) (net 11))
 (segment (start 117.5 110.5) (end 118.5 110.5) (width 0.25) (layer F.Cu) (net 11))
 (segment (start 117.05 110.05) (end 117.5 110.5) (width 0.25) (layer F.Cu) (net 11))
 (segment (start 115.5 111.95) (end 115.5 113.75) (width 0.25) (layer F.Cu) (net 7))
 (segment (start 118.75 118.25) (end 120.23 118.25) (width 0.25) (layer F.Cu) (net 7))
 (segment (start 118 117.5) (end 118.75 118.25) (width 0.25) (layer F.Cu) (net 7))
 (segment (start 118 116.25) (end 118 117.5) (width 0.25) (layer F.Cu) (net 7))
 (segment (start 115.5 113.75) (end 118 116.25) (width 0.25) (layer F.Cu) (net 7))
 (segment (start 123.25 83.5) (end 123.25 84.25) (width 0.5) (layer F.Cu) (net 10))
 (segment (start 123.25 84.25) (end 131 92) (width 0.5) (layer F.Cu) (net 10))
 (segment (start 131 92) (end 131 92.75) (width 0.5) (layer F.Cu) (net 10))
 (segment (start 131 93.75) (end 131 92.75) (width 0.5) (layer F.Cu) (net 10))
 (segment (start 129.3001 103) (end 131 101.3001) (width 0.5) (layer F.Cu) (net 10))
 (segment (start 131 93.75) (end 131 101.3001) (width 0.5) (layer F.Cu) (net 10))
 (segment (start 128 104.25) (end 127.25 105) (width 0.25) (layer F.Cu) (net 10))
 (segment (start 127.25 105) (end 127 105) (width 0.25) (layer F.Cu) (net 10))
 (segment (start 129.3001 103) (end 129.3001 102.9499) (width 0.25) (layer F.Cu) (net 10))
 (segment (start 125.3001 105) (end 127 105) (width 0.25) (layer F.Cu) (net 10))
 (segment (start 129.3001 103.6999) (end 129.3001 103) (width 0.25) (layer F.Cu) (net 10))
 (segment (start 128.75 104.25) (end 129.3001 103.6999) (width 0.25) (layer F.Cu) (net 10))
 (segment (start 128 104.25) (end 128.75 104.25) (width 0.25) (layer F.Cu) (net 10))
 (segment (start 125.3001 105) (end 125.6999 105) (width 0.25) (layer F.Cu) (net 10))
 (segment (start 121 102.5) (end 121 100.25) (width 0.25) (layer B.Cu) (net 12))
 (segment (start 120 100.25) (end 119.5 99.75) (width 0.25) (layer F.Cu) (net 12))
 (segment (start 121 100.25) (end 120 100.25) (width 0.25) (layer F.Cu) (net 12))
 (via (at 121 100.25) (size 0.6) (drill 0.4) (layers F.Cu B.Cu) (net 12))
 (segment (start 118.95 97.65) (end 118.95 99.2) (width 0.25) (layer F.Cu) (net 12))
 (segment (start 118.95 99.2) (end 119.5 99.75) (width 0.25) (layer F.Cu) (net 12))
 (segment (start 119.8001 102.75) (end 120.75 102.75) (width 0.25) (layer F.Cu) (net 12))
 (via (at 121 102.5) (size 0.6) (drill 0.4) (layers F.Cu B.Cu) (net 12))
 (segment (start 120.75 102.75) (end 121 102.5) (width 0.25) (layer F.Cu) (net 12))
 (segment (start 119.8001 104.5) (end 119.8001 102.75) (width 0.25) (layer F.Cu) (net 12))
 (segment (start 118.95 98.2) (end 118.95 97.65) (width 0.25) (layer F.Cu) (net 12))
 (segment (start 118.95 97.65) (end 118.95 98.2) (width 0.25) (layer F.Cu) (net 12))
 (segment (start 127.6999 100.75) (end 127.6999 98.35086) (width 0.25) (layer F.Cu) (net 1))
 (segment (start 127.6999 98.35086) (end 128.05 98.00076) (width 0.25) (layer F.Cu) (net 1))
 (segment (start 126.5 103) (end 126.5 103.5) (width 0.25) (layer F.Cu) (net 1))
 (segment (start 126 104) (end 125.75 104) (width 0.25) (layer F.Cu) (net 1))
 (segment (start 126.5 103.5) (end 126 104) (width 0.25) (layer F.Cu) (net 1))
 (segment (start 123.6999 103) (end 123.6999 103.4499) (width 0.25) (layer F.Cu) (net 1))
 (segment (start 123.6999 103.4499) (end 124.25 104) (width 0.25) (layer F.Cu) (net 1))
 (segment (start 126.5 101.9499) (end 127.6999 100.75) (width 0.25) (layer F.Cu) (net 1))
 (segment (start 126.5 103) (end 126.5 101.9499) (width 0.25) (layer F.Cu) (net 1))
 (segment (start 124.25 104) (end 125.75 104) (width 0.25) (layer F.Cu) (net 1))
 (segment (start 118.1999 102.75) (end 117.5 102.75) (width 0.25) (layer F.Cu) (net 13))
 (segment (start 117.05 104.2) (end 116.15 104.2) (width 0.25) (layer F.Cu) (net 13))
 (segment (start 117.25 104) (end 117.05 104.2) (width 0.25) (layer F.Cu) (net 13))
 (segment (start 117.25 103) (end 117.25 104) (width 0.25) (layer F.Cu) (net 13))
 (segment (start 117.5 102.75) (end 117.25 103) (width 0.25) (layer F.Cu) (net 13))
 (segment (start 121.75 104.4499) (end 123.1498 104.4499) (width 0.25) (layer F.Cu) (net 14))
 (segment (start 123.1498 104.4499) (end 123.6999 105) (width 0.25) (layer F.Cu) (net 14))
 (segment (start 122.97495 104.27505) (end 122.75 104.0501) (width 0.25) (layer F.Cu) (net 14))
 (segment (start 122.75 102.5) (end 121.75 101.5) (width 0.25) (layer F.Cu) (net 14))
 (segment (start 122.75 104.0501) (end 122.75 102.5) (width 0.25) (layer F.Cu) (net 14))
 (segment (start 120.5 101.5) (end 121.75 101.5) (width 0.25) (layer F.Cu) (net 14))
 (segment (start 120.5 101.5) (end 117.75 101.5) (width 0.25) (layer F.Cu) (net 14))
 (segment (start 117.75 101.5) (end 116.95 102.3) (width 0.25) (layer F.Cu) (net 14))
 (segment (start 116.95 102.3) (end 116.15 102.3) (width 0.25) (layer F.Cu) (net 14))
 (segment (start 122.97495 104.27505) (end 123.6999 105) (width 0.25) (layer F.Cu) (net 14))
 (segment (start 123.6999 107) (end 123.6999 105) (width 0.25) (layer F.Cu) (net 14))
 (segment (start 115.85 92.5) (end 115.85 90.7001) (width 0.25) (layer F.Cu) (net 18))
 (segment (start 115.85 90.7001) (end 116.0501 90.5) (width 0.25) (layer F.Cu) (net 18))
 (segment (start 115.85 92.5) (end 115.85 93.15) (width 0.5) (layer F.Cu) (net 18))
 (segment (start 112.5 96.9) (end 114.25 98.65) (width 0.5) (layer F.Cu) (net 18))
 (segment (start 112.5 94.75) (end 112.5 96.9) (width 0.5) (layer F.Cu) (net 18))
 (segment (start 113 94.25) (end 112.5 94.75) (width 0.5) (layer F.Cu) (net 18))
 (segment (start 114.75 94.25) (end 113 94.25) (width 0.5) (layer F.Cu) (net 18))
 (segment (start 115.85 93.15) (end 114.75 94.25) (width 0.5) (layer F.Cu) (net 18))
 (segment (start 114.25 98.65) (end 114.15 98.65) (width 0.25) (layer F.Cu) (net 18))
 (segment (start 118.35 109.23) (end 118.48 109.23) (width 0.25) (layer F.Cu) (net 16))
 (segment (start 118.48 109.23) (end 120.25 111) (width 0.25) (layer F.Cu) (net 16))
 (segment (start 120.25 113.05) (end 119.55 113.75) (width 0.25) (layer F.Cu) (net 16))
 (segment (start 120.25 111) (end 120.25 113.05) (width 0.25) (layer F.Cu) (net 16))
 (segment (start 119.55 113.75) (end 119.55 113.7) (width 0.25) (layer F.Cu) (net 16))
 (segment (start 124.65 110.5) (end 126 110.5) (width 0.25) (layer F.Cu) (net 15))
 (segment (start 126.5 109.1999) (end 127.6999 108) (width 0.25) (layer F.Cu) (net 15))
 (segment (start 126.5 110) (end 126.5 109.1999) (width 0.25) (layer F.Cu) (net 15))
 (segment (start 126 110.5) (end 126.5 110) (width 0.25) (layer F.Cu) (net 15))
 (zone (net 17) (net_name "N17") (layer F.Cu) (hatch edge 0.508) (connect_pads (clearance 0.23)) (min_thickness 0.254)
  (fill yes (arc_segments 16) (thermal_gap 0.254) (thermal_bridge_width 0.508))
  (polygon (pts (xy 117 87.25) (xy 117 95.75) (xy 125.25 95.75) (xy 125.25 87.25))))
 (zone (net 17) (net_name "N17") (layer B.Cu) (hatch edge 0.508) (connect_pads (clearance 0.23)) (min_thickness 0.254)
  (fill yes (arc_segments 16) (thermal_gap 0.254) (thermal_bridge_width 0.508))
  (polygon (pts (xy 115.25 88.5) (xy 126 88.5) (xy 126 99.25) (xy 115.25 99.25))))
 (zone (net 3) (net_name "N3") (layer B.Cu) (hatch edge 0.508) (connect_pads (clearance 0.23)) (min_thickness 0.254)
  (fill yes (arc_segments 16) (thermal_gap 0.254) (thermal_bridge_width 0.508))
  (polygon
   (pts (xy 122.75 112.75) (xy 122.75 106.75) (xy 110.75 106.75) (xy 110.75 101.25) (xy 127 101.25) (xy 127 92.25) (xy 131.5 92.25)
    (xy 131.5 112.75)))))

